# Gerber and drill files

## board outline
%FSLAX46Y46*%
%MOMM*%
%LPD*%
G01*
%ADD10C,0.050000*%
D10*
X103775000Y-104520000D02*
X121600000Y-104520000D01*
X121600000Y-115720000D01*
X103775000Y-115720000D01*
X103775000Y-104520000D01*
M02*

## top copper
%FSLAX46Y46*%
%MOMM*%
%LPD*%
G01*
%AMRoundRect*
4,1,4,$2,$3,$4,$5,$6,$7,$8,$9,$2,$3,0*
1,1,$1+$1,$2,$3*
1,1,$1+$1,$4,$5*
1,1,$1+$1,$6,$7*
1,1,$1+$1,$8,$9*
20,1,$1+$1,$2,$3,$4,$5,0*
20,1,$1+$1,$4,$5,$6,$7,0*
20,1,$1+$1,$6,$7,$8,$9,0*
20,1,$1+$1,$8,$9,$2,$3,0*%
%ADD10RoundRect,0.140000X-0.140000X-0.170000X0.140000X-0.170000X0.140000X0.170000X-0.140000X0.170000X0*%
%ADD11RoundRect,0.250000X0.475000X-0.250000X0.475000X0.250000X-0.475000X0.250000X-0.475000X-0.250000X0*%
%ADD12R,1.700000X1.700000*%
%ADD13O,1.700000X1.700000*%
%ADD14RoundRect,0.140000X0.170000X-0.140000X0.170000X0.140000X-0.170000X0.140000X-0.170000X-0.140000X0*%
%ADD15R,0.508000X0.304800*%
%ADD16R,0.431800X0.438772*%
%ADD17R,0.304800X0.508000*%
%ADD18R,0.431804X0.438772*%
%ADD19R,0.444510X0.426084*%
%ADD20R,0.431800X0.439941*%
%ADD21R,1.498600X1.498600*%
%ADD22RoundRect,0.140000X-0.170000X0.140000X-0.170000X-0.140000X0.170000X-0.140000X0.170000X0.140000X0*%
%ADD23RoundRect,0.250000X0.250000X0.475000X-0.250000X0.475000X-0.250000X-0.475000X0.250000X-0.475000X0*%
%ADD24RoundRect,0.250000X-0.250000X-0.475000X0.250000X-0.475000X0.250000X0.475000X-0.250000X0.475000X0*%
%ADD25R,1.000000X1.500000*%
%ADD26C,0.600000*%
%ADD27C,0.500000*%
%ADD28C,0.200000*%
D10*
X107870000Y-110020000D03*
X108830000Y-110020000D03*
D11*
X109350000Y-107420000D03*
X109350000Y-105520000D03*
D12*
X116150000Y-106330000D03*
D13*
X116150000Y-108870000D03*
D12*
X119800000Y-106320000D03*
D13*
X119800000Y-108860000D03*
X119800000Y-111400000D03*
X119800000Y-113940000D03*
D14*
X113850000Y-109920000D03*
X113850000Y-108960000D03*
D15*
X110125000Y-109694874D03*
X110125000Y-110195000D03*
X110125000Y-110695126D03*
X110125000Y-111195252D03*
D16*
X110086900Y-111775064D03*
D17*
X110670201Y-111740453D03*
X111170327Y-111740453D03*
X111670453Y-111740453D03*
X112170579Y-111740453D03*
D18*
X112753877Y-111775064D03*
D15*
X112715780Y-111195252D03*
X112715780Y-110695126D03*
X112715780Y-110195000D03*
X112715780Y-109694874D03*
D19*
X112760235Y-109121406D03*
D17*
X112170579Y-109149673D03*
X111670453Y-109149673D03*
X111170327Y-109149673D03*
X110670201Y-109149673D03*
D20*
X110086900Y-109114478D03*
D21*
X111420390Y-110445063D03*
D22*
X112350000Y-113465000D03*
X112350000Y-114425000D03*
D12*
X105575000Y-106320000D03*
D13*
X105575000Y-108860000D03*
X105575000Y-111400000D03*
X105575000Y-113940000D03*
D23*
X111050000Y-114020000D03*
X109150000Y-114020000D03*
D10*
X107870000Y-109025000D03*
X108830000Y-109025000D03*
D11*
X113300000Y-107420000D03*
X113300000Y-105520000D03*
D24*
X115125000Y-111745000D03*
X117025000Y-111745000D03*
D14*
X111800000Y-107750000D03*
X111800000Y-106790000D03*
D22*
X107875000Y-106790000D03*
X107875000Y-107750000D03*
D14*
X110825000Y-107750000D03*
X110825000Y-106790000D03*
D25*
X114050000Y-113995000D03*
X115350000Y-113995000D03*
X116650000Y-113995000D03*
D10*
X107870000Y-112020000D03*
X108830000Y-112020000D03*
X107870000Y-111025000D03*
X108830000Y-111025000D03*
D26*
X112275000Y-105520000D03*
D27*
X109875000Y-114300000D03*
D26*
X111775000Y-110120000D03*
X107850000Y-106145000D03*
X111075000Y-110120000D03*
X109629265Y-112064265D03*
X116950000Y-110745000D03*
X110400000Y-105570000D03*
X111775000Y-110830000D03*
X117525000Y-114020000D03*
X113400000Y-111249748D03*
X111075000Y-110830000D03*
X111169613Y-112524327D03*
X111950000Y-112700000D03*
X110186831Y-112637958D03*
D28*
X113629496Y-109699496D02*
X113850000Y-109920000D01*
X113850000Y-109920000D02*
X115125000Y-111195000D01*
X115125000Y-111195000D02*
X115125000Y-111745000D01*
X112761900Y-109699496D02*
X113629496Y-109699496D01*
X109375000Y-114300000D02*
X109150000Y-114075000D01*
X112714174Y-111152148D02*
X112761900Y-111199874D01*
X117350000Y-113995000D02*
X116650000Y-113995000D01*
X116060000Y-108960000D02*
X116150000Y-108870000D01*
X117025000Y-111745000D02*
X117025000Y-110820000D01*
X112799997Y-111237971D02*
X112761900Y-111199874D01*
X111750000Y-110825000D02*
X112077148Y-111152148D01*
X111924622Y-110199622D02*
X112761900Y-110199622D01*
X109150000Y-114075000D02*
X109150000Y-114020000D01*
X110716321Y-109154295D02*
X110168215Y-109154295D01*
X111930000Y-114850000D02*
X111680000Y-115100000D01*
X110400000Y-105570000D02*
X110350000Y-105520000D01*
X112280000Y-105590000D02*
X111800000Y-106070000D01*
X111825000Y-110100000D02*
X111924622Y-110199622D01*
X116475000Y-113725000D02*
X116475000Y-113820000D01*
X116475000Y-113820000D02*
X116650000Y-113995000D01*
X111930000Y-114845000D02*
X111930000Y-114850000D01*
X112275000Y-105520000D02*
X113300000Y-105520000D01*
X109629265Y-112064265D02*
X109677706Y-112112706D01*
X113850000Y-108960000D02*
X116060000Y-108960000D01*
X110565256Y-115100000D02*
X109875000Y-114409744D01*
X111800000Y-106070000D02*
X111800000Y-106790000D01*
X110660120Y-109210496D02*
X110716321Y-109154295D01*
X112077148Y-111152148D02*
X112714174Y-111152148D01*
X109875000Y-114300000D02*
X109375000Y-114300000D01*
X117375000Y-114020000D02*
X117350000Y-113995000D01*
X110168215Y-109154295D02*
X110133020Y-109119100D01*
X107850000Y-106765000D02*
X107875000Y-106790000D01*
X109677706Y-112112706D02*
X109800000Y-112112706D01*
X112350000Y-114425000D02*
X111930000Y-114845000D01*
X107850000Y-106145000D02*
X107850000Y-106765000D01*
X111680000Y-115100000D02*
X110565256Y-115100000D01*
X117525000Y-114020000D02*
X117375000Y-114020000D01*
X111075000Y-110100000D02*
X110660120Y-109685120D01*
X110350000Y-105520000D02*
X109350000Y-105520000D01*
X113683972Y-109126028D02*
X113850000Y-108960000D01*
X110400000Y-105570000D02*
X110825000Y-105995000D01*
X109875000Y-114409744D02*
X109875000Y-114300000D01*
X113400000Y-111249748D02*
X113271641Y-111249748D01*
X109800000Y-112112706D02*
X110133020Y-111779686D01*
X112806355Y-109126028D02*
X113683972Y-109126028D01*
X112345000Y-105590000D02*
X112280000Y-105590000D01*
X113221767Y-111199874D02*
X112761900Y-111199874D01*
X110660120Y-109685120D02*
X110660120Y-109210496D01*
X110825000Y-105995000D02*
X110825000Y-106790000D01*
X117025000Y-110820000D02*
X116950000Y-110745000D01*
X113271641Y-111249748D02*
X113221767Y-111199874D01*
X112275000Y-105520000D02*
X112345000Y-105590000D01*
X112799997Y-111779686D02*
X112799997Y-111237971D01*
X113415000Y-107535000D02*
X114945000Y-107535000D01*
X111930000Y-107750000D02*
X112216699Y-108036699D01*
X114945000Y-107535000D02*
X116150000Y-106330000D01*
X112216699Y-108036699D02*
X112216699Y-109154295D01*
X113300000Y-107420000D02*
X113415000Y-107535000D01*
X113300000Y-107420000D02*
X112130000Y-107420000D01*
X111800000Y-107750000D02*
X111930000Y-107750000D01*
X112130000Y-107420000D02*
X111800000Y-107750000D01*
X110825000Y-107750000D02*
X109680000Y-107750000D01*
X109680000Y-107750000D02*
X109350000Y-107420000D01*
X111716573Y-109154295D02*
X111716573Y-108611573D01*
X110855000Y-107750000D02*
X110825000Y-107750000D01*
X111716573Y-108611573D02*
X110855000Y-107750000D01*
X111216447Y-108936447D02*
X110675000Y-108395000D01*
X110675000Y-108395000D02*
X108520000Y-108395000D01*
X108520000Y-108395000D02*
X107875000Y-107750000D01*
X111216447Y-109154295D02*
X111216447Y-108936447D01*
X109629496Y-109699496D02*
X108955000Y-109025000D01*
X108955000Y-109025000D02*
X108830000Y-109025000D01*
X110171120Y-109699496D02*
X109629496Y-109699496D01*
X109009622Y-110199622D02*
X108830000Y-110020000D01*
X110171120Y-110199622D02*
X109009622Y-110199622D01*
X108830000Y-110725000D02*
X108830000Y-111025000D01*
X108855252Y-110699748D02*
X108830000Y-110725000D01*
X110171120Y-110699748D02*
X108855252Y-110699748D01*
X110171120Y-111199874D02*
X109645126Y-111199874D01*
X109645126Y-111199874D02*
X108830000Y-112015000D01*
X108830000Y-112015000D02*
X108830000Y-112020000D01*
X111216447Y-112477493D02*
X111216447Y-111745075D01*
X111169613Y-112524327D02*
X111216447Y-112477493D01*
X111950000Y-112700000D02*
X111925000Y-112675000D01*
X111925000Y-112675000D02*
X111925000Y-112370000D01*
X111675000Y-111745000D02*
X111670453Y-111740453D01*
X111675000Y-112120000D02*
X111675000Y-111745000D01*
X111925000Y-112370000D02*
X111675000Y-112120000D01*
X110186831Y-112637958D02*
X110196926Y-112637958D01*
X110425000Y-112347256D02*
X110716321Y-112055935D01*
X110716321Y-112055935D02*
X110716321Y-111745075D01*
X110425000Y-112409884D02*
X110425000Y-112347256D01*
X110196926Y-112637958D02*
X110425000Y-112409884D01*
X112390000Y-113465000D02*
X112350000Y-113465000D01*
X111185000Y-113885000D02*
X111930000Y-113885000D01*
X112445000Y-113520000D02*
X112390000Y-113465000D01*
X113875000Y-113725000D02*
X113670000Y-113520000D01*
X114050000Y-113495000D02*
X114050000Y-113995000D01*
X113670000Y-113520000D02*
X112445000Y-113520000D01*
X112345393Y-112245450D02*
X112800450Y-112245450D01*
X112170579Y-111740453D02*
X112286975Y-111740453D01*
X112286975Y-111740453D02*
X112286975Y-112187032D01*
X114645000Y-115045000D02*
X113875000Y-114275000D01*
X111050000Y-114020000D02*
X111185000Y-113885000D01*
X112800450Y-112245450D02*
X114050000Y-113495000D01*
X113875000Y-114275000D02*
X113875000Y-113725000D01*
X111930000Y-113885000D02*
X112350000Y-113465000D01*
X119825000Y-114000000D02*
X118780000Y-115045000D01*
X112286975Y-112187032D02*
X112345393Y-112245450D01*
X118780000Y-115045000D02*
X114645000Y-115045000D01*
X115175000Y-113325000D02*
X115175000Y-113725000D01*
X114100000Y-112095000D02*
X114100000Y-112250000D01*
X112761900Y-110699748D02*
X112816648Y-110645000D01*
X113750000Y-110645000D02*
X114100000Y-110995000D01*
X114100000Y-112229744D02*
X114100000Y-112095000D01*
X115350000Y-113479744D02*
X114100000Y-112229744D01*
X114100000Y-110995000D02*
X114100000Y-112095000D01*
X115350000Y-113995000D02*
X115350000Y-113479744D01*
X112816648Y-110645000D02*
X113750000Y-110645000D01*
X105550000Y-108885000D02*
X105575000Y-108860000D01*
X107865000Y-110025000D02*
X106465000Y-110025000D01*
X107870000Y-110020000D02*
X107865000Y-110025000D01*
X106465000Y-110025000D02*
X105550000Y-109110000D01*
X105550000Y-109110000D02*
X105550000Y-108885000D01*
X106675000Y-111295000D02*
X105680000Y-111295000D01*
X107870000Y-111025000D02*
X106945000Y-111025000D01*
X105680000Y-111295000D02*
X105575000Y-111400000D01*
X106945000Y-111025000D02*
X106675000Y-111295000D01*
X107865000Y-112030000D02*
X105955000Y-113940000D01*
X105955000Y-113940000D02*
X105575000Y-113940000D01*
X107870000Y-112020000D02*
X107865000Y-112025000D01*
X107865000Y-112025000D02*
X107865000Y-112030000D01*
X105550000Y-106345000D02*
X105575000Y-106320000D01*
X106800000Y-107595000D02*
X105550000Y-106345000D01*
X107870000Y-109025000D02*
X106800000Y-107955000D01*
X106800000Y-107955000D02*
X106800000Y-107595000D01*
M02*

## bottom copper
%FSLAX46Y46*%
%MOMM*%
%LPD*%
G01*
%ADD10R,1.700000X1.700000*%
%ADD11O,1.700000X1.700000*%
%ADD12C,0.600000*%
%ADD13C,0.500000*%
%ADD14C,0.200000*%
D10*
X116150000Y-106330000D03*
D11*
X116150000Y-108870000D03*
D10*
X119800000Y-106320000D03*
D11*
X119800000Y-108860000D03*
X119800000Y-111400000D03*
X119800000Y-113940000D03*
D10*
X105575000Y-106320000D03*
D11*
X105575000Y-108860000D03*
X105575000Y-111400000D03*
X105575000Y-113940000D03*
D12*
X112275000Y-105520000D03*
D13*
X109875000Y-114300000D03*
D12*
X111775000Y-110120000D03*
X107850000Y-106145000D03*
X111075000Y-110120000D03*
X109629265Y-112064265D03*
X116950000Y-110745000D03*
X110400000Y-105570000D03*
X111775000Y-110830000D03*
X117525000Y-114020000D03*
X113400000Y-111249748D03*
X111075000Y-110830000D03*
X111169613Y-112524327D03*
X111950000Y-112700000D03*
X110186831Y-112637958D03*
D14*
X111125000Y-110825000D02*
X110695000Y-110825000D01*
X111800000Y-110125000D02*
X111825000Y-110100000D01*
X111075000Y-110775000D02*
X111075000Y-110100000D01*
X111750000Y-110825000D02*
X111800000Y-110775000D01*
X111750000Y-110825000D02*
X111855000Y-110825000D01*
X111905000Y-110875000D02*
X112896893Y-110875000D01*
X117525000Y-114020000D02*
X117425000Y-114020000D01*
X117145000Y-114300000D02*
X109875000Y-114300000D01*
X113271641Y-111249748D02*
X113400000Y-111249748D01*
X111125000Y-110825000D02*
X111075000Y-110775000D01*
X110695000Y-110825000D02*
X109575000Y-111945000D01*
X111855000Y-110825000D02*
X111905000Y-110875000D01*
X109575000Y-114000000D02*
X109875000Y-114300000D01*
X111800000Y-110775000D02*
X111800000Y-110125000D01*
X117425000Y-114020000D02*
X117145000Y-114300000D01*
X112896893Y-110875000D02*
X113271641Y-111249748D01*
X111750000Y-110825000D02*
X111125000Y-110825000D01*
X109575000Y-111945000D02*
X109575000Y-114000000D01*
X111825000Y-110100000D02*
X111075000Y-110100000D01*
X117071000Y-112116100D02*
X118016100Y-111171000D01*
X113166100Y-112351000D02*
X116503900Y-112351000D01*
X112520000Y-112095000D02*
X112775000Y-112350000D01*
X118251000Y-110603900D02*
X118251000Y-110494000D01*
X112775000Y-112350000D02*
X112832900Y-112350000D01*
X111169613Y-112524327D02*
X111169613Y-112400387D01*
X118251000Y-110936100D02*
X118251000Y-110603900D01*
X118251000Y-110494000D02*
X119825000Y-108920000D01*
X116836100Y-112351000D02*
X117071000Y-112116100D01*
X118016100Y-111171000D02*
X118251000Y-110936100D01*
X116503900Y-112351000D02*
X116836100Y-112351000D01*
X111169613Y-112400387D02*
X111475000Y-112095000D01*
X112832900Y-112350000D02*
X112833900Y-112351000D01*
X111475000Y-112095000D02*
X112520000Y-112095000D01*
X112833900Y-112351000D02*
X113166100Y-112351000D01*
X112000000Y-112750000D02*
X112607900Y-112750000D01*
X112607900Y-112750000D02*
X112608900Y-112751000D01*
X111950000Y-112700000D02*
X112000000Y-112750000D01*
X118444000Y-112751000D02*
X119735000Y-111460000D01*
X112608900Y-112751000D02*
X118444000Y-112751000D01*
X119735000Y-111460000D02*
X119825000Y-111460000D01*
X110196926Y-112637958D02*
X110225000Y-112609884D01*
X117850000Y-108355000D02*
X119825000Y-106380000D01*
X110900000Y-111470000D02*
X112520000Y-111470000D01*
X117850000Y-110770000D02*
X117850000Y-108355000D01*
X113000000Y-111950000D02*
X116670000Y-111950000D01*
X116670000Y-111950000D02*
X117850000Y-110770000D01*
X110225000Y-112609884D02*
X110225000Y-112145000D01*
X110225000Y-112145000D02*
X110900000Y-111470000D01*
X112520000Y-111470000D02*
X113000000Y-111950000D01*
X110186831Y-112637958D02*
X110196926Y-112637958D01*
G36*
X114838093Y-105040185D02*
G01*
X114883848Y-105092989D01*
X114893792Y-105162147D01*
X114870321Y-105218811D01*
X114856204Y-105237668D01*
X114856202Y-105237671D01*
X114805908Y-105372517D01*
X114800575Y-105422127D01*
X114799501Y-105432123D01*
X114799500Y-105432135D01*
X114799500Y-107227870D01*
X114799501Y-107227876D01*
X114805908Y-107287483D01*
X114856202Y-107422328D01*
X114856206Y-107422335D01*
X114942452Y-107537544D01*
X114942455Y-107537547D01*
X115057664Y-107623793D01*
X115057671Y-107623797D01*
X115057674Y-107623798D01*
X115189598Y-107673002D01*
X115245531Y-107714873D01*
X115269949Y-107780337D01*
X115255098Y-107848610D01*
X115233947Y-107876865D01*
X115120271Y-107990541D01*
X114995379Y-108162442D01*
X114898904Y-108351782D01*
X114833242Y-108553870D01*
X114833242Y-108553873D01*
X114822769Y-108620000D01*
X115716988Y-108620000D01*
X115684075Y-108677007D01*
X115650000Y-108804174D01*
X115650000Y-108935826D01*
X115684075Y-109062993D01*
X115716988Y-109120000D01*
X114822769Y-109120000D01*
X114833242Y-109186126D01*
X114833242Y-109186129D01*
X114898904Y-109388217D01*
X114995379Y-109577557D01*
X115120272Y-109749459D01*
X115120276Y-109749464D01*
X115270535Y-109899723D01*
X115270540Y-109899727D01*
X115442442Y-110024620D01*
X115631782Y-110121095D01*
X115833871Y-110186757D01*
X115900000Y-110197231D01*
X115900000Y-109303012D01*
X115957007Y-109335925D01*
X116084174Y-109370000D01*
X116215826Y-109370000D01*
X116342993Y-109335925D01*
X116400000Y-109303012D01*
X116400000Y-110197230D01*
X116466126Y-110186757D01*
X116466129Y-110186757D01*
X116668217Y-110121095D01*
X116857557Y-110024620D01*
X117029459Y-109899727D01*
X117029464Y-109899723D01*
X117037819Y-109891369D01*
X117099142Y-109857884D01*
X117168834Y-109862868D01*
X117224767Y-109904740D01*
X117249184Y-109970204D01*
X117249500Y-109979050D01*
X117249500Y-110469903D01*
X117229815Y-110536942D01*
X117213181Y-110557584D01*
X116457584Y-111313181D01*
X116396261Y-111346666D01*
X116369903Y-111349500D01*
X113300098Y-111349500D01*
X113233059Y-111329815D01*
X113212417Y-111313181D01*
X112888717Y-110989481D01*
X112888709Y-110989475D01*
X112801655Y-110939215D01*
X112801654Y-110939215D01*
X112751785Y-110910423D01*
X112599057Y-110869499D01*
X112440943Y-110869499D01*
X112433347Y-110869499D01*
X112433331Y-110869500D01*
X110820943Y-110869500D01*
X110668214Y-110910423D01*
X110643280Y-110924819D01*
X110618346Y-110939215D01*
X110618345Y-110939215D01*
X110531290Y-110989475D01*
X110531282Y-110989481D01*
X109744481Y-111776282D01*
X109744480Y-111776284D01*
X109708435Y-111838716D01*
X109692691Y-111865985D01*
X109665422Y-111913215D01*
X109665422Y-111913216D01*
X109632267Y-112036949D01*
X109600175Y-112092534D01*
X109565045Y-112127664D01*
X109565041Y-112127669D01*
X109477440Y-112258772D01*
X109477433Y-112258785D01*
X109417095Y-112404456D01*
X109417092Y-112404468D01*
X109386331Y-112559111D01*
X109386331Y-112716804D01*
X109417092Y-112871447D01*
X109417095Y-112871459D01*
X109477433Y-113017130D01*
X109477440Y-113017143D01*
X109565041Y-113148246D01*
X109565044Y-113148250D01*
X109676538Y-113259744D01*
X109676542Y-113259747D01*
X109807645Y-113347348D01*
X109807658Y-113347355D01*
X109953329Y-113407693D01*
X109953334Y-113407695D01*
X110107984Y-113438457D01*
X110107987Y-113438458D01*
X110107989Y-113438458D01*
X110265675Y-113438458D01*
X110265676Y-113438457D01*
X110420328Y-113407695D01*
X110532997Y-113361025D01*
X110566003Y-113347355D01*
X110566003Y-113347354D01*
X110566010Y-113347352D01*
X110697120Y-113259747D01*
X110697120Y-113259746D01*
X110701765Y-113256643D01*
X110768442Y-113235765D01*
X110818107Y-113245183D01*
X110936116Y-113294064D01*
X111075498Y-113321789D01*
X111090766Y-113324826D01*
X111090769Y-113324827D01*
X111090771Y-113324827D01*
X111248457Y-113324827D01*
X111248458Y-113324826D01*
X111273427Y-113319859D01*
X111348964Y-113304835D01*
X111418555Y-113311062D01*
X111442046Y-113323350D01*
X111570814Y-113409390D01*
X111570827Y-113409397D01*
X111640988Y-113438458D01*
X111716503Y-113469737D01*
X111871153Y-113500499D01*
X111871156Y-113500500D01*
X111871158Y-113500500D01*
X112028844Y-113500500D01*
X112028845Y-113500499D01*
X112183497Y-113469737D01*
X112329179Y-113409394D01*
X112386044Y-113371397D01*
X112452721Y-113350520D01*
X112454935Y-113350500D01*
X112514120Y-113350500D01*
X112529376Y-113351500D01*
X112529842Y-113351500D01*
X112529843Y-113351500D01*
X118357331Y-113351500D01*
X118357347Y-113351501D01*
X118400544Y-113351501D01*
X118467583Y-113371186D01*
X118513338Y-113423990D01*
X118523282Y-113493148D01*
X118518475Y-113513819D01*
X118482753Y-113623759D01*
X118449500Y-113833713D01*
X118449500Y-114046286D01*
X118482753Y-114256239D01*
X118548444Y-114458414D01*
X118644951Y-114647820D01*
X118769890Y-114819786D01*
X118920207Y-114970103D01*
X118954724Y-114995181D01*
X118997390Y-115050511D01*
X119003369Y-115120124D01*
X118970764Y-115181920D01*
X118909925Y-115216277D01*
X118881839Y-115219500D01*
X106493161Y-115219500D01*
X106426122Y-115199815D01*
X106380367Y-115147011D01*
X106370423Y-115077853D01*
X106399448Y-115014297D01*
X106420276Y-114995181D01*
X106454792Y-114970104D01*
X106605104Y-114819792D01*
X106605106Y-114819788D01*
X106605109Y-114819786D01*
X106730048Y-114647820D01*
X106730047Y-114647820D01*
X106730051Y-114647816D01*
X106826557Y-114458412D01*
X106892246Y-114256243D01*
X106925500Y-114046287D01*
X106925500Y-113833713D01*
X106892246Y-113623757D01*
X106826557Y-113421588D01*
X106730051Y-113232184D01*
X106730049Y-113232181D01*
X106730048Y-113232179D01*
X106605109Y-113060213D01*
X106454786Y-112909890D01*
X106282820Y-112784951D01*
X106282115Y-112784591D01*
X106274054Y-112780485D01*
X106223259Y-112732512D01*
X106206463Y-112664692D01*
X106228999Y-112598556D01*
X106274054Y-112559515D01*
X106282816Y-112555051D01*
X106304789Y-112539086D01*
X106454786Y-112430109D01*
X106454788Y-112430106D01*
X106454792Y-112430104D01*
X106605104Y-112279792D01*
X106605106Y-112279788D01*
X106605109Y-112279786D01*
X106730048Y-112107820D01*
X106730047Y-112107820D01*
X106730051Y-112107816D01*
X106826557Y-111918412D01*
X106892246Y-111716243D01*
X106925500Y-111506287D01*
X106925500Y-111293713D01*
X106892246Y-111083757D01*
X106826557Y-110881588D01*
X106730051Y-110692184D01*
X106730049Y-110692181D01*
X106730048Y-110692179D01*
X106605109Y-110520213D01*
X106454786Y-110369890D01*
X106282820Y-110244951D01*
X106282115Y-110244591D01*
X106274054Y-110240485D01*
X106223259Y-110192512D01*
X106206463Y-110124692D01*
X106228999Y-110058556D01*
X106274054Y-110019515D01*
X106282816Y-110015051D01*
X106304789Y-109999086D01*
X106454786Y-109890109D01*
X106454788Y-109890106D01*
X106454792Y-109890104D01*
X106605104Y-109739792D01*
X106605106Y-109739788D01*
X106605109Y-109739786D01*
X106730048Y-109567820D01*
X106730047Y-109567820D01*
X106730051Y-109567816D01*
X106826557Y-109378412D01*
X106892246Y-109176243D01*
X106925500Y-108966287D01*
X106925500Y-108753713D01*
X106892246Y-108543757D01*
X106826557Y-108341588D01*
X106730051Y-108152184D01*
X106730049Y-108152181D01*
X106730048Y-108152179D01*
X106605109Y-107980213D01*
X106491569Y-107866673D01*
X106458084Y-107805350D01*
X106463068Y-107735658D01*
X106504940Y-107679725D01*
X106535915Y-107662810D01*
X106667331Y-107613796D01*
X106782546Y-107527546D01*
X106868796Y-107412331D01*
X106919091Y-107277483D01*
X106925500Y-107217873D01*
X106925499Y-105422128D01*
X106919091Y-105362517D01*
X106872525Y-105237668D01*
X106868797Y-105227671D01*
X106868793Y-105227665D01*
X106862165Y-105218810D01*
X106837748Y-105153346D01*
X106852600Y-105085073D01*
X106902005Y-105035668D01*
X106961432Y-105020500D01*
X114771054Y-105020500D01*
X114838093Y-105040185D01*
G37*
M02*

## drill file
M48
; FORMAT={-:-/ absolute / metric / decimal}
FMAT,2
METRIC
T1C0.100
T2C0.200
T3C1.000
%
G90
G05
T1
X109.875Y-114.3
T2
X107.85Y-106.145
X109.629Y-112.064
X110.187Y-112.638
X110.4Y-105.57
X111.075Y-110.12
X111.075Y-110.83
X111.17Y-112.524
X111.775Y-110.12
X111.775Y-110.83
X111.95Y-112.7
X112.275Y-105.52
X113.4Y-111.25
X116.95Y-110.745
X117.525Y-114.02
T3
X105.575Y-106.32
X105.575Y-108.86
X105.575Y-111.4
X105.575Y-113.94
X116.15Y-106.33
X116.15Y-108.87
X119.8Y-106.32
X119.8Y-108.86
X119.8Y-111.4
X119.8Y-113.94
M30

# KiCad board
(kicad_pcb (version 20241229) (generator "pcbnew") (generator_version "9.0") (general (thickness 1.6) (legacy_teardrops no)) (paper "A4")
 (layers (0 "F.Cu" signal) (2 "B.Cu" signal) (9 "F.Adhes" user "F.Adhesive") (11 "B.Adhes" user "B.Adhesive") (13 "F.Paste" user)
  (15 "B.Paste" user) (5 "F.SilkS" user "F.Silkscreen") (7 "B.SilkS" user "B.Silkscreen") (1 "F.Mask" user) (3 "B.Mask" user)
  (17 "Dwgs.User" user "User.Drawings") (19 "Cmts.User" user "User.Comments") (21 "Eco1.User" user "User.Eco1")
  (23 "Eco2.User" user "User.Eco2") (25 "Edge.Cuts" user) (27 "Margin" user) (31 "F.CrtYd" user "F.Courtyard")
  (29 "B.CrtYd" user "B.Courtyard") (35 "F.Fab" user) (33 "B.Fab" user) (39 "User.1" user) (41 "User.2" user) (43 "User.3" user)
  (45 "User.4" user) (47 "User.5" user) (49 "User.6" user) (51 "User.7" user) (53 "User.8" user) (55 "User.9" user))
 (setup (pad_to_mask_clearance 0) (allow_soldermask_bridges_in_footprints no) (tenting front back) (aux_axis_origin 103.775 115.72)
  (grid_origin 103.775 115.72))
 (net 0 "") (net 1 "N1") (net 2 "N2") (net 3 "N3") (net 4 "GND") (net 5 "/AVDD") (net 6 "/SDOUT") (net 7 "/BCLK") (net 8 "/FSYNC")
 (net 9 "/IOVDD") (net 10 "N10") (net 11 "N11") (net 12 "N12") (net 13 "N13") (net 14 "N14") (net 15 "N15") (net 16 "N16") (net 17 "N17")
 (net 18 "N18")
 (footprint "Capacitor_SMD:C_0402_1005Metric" (layer "F.Cu") (at 108.35 110.02)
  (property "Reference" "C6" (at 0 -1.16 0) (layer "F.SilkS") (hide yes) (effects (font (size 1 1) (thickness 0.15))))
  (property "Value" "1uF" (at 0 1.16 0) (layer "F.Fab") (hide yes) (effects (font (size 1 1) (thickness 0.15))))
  (pad "1" smd roundrect (at -0.48 0) (size 0.56 0.62) (layers "F.Cu" "F.Mask" "F.Paste") (roundrect_rratio 0.25) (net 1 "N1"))
  (pad "2" smd roundrect (at 0.48 0) (size 0.56 0.62) (layers "F.Cu" "F.Mask" "F.Paste") (roundrect_rratio 0.25) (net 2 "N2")))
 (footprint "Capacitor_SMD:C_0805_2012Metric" (layer "F.Cu") (at 109.35 106.47 90)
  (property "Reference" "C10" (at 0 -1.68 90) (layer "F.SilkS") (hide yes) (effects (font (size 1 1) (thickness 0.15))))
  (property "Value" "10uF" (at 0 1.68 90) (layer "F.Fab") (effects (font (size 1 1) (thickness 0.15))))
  (pad "1" smd roundrect (at -0.95 0 90) (size 1 1.45) (layers "F.Cu" "F.Mask" "F.Paste") (roundrect_rratio 0.25) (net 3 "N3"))
  (pad "2" smd roundrect (at 0.95 0 90) (size 1 1.45) (layers "F.Cu" "F.Mask" "F.Paste") (roundrect_rratio 0.25) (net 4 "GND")))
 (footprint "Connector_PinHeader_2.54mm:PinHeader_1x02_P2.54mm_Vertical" (layer "F.Cu") (at 116.15 106.33)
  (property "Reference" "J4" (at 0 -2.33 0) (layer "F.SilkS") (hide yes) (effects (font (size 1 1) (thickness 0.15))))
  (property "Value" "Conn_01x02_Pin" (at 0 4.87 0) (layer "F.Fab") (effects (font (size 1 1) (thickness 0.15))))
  (pad "1" thru_hole rect (at 0 0) (size 1.7 1.7) (drill 1) (layers "*.Cu" "*.Mask") (remove_unused_layers no) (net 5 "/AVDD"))
  (pad "2" thru_hole oval (at 0 2.54) (size 1.7 1.7) (drill 1) (layers "*.Cu" "*.Mask") (remove_unused_layers no) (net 4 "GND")))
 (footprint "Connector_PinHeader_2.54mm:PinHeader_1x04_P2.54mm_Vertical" (layer "F.Cu") (at 119.8 106.32)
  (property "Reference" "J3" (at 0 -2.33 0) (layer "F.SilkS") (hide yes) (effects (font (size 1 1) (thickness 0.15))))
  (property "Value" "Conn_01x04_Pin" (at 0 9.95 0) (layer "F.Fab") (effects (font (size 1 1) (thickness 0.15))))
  (pad "1" thru_hole rect (at 0 0) (size 1.7 1.7) (drill 1) (layers "*.Cu" "*.Mask") (remove_unused_layers no) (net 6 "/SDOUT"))
  (pad "2" thru_hole oval (at 0 2.54) (size 1.7 1.7) (drill 1) (layers "*.Cu" "*.Mask") (remove_unused_layers no) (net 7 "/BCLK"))
  (pad "3" thru_hole oval (at 0 5.08) (size 1.7 1.7) (drill 1) (layers "*.Cu" "*.Mask") (remove_unused_layers no) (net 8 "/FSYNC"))
  (pad "4" thru_hole oval (at 0 7.62) (size 1.7 1.7) (drill 1) (layers "*.Cu" "*.Mask") (remove_unused_layers no) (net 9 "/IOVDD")))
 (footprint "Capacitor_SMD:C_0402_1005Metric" (layer "F.Cu") (at 113.85 109.44 90)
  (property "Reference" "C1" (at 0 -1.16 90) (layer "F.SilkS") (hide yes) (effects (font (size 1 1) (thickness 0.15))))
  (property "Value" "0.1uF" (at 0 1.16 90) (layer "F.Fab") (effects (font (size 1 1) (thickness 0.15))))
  (pad "1" smd roundrect (at -0.48 0 90) (size 0.56 0.62) (layers "F.Cu" "F.Mask" "F.Paste") (roundrect_rratio 0.25) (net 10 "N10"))
  (pad "2" smd roundrect (at 0.48 0 90) (size 0.56 0.62) (layers "F.Cu" "F.Mask" "F.Paste") (roundrect_rratio 0.25) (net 4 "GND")))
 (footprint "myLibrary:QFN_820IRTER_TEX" (layer "F.Cu") (at 111.42039 110.445063)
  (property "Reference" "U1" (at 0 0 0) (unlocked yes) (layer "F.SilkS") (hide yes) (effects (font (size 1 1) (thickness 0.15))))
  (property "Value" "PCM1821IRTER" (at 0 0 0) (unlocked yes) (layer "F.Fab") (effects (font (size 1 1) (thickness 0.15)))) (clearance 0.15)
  (pad "1" smd rect (at -1.29539 -0.750189 90) (size 0.3048 0.508) (layers "F.Cu" "F.Mask" "F.Paste") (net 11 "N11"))
  (pad "2" smd rect (at -1.29539 -0.250063 90) (size 0.3048 0.508) (layers "F.Cu" "F.Mask" "F.Paste") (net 2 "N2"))
  (pad "3" smd rect (at -1.29539 0.250063 90) (size 0.3048 0.508) (layers "F.Cu" "F.Mask" "F.Paste") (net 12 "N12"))
  (pad "4" smd rect (at -1.29539 0.750189 90) (size 0.3048 0.508) (layers "F.Cu" "F.Mask" "F.Paste") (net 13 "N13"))
  (pad "5" smd rect (at -1.33349 1.330001 90) (size 0.438772 0.4318) (layers "F.Cu" "F.Mask" "F.Paste") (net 4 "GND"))
  (pad "6" smd rect (at -0.750189 1.29539) (size 0.3048 0.508) (layers "F.Cu" "F.Mask" "F.Paste") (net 6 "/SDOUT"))
  (pad "7" smd rect (at -0.250063 1.29539) (size 0.3048 0.508) (layers "F.Cu" "F.Mask" "F.Paste") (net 7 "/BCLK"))
  (pad "8" smd rect (at 0.250063 1.29539) (size 0.3048 0.508) (layers "F.Cu" "F.Mask" "F.Paste") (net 8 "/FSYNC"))
  (pad "9" smd rect (at 0.750189 1.29539) (size 0.3048 0.508) (layers "F.Cu" "F.Mask" "F.Paste") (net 9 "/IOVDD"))
  (pad "10" smd rect (at 1.333487 1.330001 90) (size 0.438772 0.431804) (layers "F.Cu" "F.Mask" "F.Paste") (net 4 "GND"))
  (pad "11" smd rect (at 1.29539 0.750189 90) (size 0.3048 0.508) (layers "F.Cu" "F.Mask" "F.Paste") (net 4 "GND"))
  (pad "12" smd rect (at 1.29539 0.250063 90) (size 0.3048 0.508) (layers "F.Cu" "F.Mask" "F.Paste") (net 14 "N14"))
  (pad "13" smd rect (at 1.29539 -0.250063 90) (size 0.3048 0.508) (layers "F.Cu" "F.Mask" "F.Paste") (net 4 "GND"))
  (pad "14" smd rect (at 1.29539 -0.750189 90) (size 0.3048 0.508) (layers "F.Cu" "F.Mask" "F.Paste") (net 10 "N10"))
  (pad "15" smd rect (at 1.339845 -1.323657 90) (size 0.426084 0.44451) (layers "F.Cu" "F.Mask" "F.Paste") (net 4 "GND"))
  (pad "16" smd rect (at 0.750189 -1.29539) (size 0.3048 0.508) (layers "F.Cu" "F.Mask" "F.Paste") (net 5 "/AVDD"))
  (pad "17" smd rect (at 0.250063 -1.29539) (size 0.3048 0.508) (layers "F.Cu" "F.Mask" "F.Paste") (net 3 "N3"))
  (pad "18" smd rect (at -0.250063 -1.29539) (size 0.3048 0.508) (layers "F.Cu" "F.Mask" "F.Paste") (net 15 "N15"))
  (pad "19" smd rect (at -0.750189 -1.29539) (size 0.3048 0.508) (layers "F.Cu" "F.Mask" "F.Paste") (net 4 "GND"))
  (pad "20" smd rect (at -1.33349 -1.330585 90) (size 0.439941 0.4318) (layers "F.Cu" "F.Mask" "F.Paste") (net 4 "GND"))
  (pad "21" smd rect (at 0 0) (size 1.4986 1.4986) (layers "F.Cu" "F.Mask" "F.Paste") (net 4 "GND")))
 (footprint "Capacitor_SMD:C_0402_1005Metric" (layer "F.Cu") (at 112.35 113.945 -90)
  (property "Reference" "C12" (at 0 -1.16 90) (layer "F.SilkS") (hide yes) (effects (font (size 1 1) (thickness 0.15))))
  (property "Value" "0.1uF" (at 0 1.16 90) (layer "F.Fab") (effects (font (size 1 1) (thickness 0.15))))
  (pad "1" smd roundrect (at -0.48 0 270) (size 0.56 0.62) (layers "F.Cu" "F.Mask" "F.Paste") (roundrect_rratio 0.25) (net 9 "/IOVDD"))
  (pad "2" smd roundrect (at 0.48 0 270) (size 0.56 0.62) (layers "F.Cu" "F.Mask" "F.Paste") (roundrect_rratio 0.25) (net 4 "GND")))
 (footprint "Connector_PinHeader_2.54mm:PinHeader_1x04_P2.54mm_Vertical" (layer "F.Cu") (at 105.575 106.32)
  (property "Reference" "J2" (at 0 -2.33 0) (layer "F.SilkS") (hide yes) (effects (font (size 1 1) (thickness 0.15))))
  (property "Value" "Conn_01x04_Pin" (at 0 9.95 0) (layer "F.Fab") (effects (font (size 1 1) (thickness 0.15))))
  (pad "1" thru_hole rect (at 0 0) (size 1.7 1.7) (drill 1) (layers "*.Cu" "*.Mask") (remove_unused_layers no) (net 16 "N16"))
  (pad "2" thru_hole oval (at 0 2.54) (size 1.7 1.7) (drill 1) (layers "*.Cu" "*.Mask") (remove_unused_layers no) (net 1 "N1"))
  (pad "3" thru_hole oval (at 0 5.08) (size 1.7 1.7) (drill 1) (layers "*.Cu" "*.Mask") (remove_unused_layers no) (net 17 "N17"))
  (pad "4" thru_hole oval (at 0 7.62) (size 1.7 1.7) (drill 1) (layers "*.Cu" "*.Mask") (remove_unused_layers no) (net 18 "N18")))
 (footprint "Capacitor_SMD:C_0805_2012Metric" (layer "F.Cu") (at 110.1 114.02 180)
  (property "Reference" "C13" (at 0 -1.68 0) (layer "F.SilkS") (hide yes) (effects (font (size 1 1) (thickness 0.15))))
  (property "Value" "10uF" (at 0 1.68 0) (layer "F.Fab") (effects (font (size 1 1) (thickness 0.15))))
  (pad "1" smd roundrect (at -0.95 0 180) (size 1 1.45) (layers "F.Cu" "F.Mask" "F.Paste") (roundrect_rratio 0.25) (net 9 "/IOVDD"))
  (pad "2" smd roundrect (at 0.95 0 180) (size 1 1.45) (layers "F.Cu" "F.Mask" "F.Paste") (roundrect_rratio 0.25) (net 4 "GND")))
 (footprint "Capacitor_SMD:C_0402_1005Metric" (layer "F.Cu") (at 108.35 109.025)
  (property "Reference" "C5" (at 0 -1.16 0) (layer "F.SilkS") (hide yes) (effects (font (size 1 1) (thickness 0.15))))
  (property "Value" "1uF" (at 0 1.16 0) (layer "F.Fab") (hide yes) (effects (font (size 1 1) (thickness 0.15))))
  (pad "1" smd roundrect (at -0.48 0) (size 0.56 0.62) (layers "F.Cu" "F.Mask" "F.Paste") (roundrect_rratio 0.25) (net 16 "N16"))
  (pad "2" smd roundrect (at 0.48 0) (size 0.56 0.62) (layers "F.Cu" "F.Mask" "F.Paste") (roundrect_rratio 0.25) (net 11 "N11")))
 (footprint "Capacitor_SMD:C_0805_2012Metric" (layer "F.Cu") (at 113.3 106.47 90)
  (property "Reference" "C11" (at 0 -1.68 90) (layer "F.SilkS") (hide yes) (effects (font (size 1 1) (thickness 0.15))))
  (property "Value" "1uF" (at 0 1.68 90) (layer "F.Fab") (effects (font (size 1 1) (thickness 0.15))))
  (pad "1" smd roundrect (at -0.95 0 90) (size 1 1.45) (layers "F.Cu" "F.Mask" "F.Paste") (roundrect_rratio 0.25) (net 5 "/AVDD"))
  (pad "2" smd roundrect (at 0.95 0 90) (size 1 1.45) (layers "F.Cu" "F.Mask" "F.Paste") (roundrect_rratio 0.25) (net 4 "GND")))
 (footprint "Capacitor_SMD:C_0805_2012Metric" (layer "F.Cu") (at 116.075 111.745)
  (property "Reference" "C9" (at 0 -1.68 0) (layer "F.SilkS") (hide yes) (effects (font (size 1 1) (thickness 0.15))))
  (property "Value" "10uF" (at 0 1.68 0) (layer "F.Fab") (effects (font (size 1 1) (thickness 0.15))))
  (pad "1" smd roundrect (at -0.95 0) (size 1 1.45) (layers "F.Cu" "F.Mask" "F.Paste") (roundrect_rratio 0.25) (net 10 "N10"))
  (pad "2" smd roundrect (at 0.95 0) (size 1 1.45) (layers "F.Cu" "F.Mask" "F.Paste") (roundrect_rratio 0.25) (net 4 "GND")))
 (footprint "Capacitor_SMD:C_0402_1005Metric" (layer "F.Cu") (at 111.8 107.27 90)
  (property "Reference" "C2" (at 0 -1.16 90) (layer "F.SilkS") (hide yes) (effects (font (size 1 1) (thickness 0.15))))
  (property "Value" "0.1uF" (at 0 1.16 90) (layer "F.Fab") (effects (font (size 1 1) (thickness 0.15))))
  (pad "1" smd roundrect (at -0.48 0 90) (size 0.56 0.62) (layers "F.Cu" "F.Mask" "F.Paste") (roundrect_rratio 0.25) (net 5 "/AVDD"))
  (pad "2" smd roundrect (at 0.48 0 90) (size 0.56 0.62) (layers "F.Cu" "F.Mask" "F.Paste") (roundrect_rratio 0.25) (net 4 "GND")))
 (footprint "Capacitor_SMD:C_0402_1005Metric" (layer "F.Cu") (at 107.875 107.27 -90)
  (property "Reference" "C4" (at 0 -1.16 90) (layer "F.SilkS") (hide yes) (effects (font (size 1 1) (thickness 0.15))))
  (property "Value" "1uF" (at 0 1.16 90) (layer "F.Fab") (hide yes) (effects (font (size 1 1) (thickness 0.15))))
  (pad "1" smd roundrect (at -0.48 0 270) (size 0.56 0.62) (layers "F.Cu" "F.Mask" "F.Paste") (roundrect_rratio 0.25) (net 4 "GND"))
  (pad "2" smd roundrect (at 0.48 0 270) (size 0.56 0.62) (layers "F.Cu" "F.Mask" "F.Paste") (roundrect_rratio 0.25) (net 15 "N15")))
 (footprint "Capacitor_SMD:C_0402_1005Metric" (layer "F.Cu") (at 110.825 107.27 90)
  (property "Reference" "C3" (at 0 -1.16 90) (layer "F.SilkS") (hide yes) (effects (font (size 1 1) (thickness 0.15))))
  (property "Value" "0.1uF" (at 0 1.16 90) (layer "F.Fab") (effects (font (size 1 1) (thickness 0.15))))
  (pad "1" smd roundrect (at -0.48 0 90) (size 0.56 0.62) (layers "F.Cu" "F.Mask" "F.Paste") (roundrect_rratio 0.25) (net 3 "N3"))
  (pad "2" smd roundrect (at 0.48 0 90) (size 0.56 0.62) (layers "F.Cu" "F.Mask" "F.Paste") (roundrect_rratio 0.25) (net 4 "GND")))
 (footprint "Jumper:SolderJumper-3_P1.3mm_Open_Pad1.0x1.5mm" (layer "F.Cu") (at 115.35 113.995)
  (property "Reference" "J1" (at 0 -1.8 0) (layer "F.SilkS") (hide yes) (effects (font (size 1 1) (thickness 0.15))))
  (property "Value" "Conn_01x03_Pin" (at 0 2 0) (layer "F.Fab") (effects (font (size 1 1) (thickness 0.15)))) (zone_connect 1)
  (pad "1" smd rect (at -1.3 0) (size 1 1.5) (layers "F.Cu" "F.Mask") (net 9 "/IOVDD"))
  (pad "2" smd rect (at 0 0) (size 1 1.5) (layers "F.Cu" "F.Mask") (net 14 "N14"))
  (pad "3" smd rect (at 1.3 0) (size 1 1.5) (layers "F.Cu" "F.Mask") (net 4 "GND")))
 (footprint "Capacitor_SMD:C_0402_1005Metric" (layer "F.Cu") (at 108.35 112.02)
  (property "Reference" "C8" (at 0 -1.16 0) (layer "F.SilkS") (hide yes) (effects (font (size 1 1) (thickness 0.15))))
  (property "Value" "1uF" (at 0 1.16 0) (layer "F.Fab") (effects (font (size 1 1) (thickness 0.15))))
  (pad "1" smd roundrect (at -0.48 0) (size 0.56 0.62) (layers "F.Cu" "F.Mask" "F.Paste") (roundrect_rratio 0.25) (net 18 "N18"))
  (pad "2" smd roundrect (at 0.48 0) (size 0.56 0.62) (layers "F.Cu" "F.Mask" "F.Paste") (roundrect_rratio 0.25) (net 13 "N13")))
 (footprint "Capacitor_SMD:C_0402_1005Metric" (layer "F.Cu") (at 108.35 111.025)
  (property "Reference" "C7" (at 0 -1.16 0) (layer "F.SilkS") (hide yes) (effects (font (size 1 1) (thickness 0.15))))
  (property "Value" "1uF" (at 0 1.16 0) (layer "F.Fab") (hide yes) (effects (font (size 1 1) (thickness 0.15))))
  (pad "1" smd roundrect (at -0.48 0) (size 0.56 0.62) (layers "F.Cu" "F.Mask" "F.Paste") (roundrect_rratio 0.25) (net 17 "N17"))
  (pad "2" smd roundrect (at 0.48 0) (size 0.56 0.62) (layers "F.Cu" "F.Mask" "F.Paste") (roundrect_rratio 0.25) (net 12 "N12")))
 (gr_rect (start 103.775 104.52) (end 121.6 115.72) (stroke (width 0.05) (type default)) (fill no) (layer "Edge.Cuts"))
 (segment (start 113.629496 109.699496) (end 113.85 109.92) (width 0.2) (layer "F.Cu") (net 10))
 (segment (start 113.85 109.92) (end 115.125 111.195) (width 0.2) (layer "F.Cu") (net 10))
 (segment (start 115.125 111.195) (end 115.125 111.745) (width 0.2) (layer "F.Cu") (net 10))
 (segment (start 112.7619 109.699496) (end 113.629496 109.699496) (width 0.2) (layer "F.Cu") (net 10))
 (segment (start 109.375 114.3) (end 109.15 114.075) (width 0.2) (layer "F.Cu") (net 4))
 (segment (start 112.714174 111.152148) (end 112.7619 111.199874) (width 0.2) (layer "F.Cu") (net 4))
 (segment (start 117.35 113.995) (end 116.65 113.995) (width 0.2) (layer "F.Cu") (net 4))
 (segment (start 116.06 108.96) (end 116.15 108.87) (width 0.2) (layer "F.Cu") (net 4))
 (segment (start 117.025 111.745) (end 117.025 110.82) (width 0.2) (layer "F.Cu") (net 4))
 (segment (start 112.799997 111.237971) (end 112.7619 111.199874) (width 0.2) (layer "F.Cu") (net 4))
 (segment (start 111.75 110.825) (end 112.077148 111.152148) (width 0.2) (layer "F.Cu") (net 4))
 (segment (start 111.924622 110.199622) (end 112.7619 110.199622) (width 0.2) (layer "F.Cu") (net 4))
 (segment (start 109.15 114.075) (end 109.15 114.02) (width 0.2) (layer "F.Cu") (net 4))
 (segment (start 110.716321 109.154295) (end 110.168215 109.154295) (width 0.2) (layer "F.Cu") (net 4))
 (segment (start 111.93 114.85) (end 111.68 115.1) (width 0.2) (layer "F.Cu") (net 4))
 (segment (start 110.4 105.57) (end 110.35 105.52) (width 0.2) (layer "F.Cu") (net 4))
 (segment (start 112.28 105.59) (end 111.8 106.07) (width 0.2) (layer "F.Cu") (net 4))
 (segment (start 111.825 110.1) (end 111.924622 110.199622) (width 0.2) (layer "F.Cu") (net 4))
 (segment (start 116.475 113.725) (end 116.475 113.82) (width 0.2) (layer "F.Cu") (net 4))
 (segment (start 116.475 113.82) (end 116.65 113.995) (width 0.2) (layer "F.Cu") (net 4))
 (segment (start 111.93 114.845) (end 111.93 114.85) (width 0.2) (layer "F.Cu") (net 4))
 (segment (start 112.275 105.52) (end 113.3 105.52) (width 0.2) (layer "F.Cu") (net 4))
 (segment (start 109.629265 112.064265) (end 109.677706 112.112706) (width 0.2) (layer "F.Cu") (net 4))
 (segment (start 113.85 108.96) (end 116.06 108.96) (width 0.2) (layer "F.Cu") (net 4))
 (segment (start 110.565256 115.1) (end 109.875 114.409744) (width 0.2) (layer "F.Cu") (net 4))
 (segment (start 111.8 106.07) (end 111.8 106.79) (width 0.2) (layer "F.Cu") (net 4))
 (segment (start 110.66012 109.210496) (end 110.716321 109.154295) (width 0.2) (layer "F.Cu") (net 4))
 (segment (start 112.077148 111.152148) (end 112.714174 111.152148) (width 0.2) (layer "F.Cu") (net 4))
 (segment (start 109.875 114.3) (end 109.375 114.3) (width 0.2) (layer "F.Cu") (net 4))
 (segment (start 117.375 114.02) (end 117.35 113.995) (width 0.2) (layer "F.Cu") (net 4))
 (segment (start 110.168215 109.154295) (end 110.13302 109.1191) (width 0.2) (layer "F.Cu") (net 4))
 (segment (start 107.85 106.765) (end 107.875 106.79) (width 0.2) (layer "F.Cu") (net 4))
 (segment (start 109.677706 112.112706) (end 109.8 112.112706) (width 0.2) (layer "F.Cu") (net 4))
 (segment (start 112.35 114.425) (end 111.93 114.845) (width 0.2) (layer "F.Cu") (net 4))
 (segment (start 107.85 106.145) (end 107.85 106.765) (width 0.2) (layer "F.Cu") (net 4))
 (segment (start 111.68 115.1) (end 110.565256 115.1) (width 0.2) (layer "F.Cu") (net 4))
 (segment (start 117.525 114.02) (end 117.375 114.02) (width 0.2) (layer "F.Cu") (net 4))
 (segment (start 111.075 110.1) (end 110.66012 109.68512) (width 0.2) (layer "F.Cu") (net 4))
 (segment (start 110.35 105.52) (end 109.35 105.52) (width 0.2) (layer "F.Cu") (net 4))
 (segment (start 113.683972 109.126028) (end 113.85 108.96) (width 0.2) (layer "F.Cu") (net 4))
 (segment (start 110.4 105.57) (end 110.825 105.995) (width 0.2) (layer "F.Cu") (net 4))
 (segment (start 109.875 114.409744) (end 109.875 114.3) (width 0.2) (layer "F.Cu") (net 4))
 (segment (start 113.4 111.249748) (end 113.271641 111.249748) (width 0.2) (layer "F.Cu") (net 4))
 (segment (start 109.8 112.112706) (end 110.13302 111.779686) (width 0.2) (layer "F.Cu") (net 4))
 (segment (start 112.806355 109.126028) (end 113.683972 109.126028) (width 0.2) (layer "F.Cu") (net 4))
 (segment (start 112.345 105.59) (end 112.28 105.59) (width 0.2) (layer "F.Cu") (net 4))
 (segment (start 113.221767 111.199874) (end 112.7619 111.199874) (width 0.2) (layer "F.Cu") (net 4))
 (segment (start 110.66012 109.68512) (end 110.66012 109.210496) (width 0.2) (layer "F.Cu") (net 4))
 (segment (start 110.825 105.995) (end 110.825 106.79) (width 0.2) (layer "F.Cu") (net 4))
 (segment (start 117.025 110.82) (end 116.95 110.745) (width 0.2) (layer "F.Cu") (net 4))
 (segment (start 113.271641 111.249748) (end 113.221767 111.199874) (width 0.2) (layer "F.Cu") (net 4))
 (segment (start 112.275 105.52) (end 112.345 105.59) (width 0.2) (layer "F.Cu") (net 4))
 (segment (start 112.799997 111.779686) (end 112.799997 111.237971) (width 0.2) (layer "F.Cu") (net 4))
 (via (at 112.275 105.52) (size 0.6) (drill 0.2) (layers "F.Cu" "B.Cu") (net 4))
 (via (at 109.875 114.3) (size 0.5) (drill 0.1) (layers "F.Cu" "B.Cu") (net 4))
 (via (at 111.775 110.12) (size 0.6) (drill 0.2) (layers "F.Cu" "B.Cu") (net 4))
 (via (at 107.85 106.145) (size 0.6) (drill 0.2) (layers "F.Cu" "B.Cu") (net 4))
 (via (at 111.075 110.12) (size 0.6) (drill 0.2) (layers "F.Cu" "B.Cu") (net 4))
 (via (at 109.629265 112.064265) (size 0.6) (drill 0.2) (layers "F.Cu" "B.Cu") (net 4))
 (via (at 116.95 110.745) (size 0.6) (drill 0.2) (layers "F.Cu" "B.Cu") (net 4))
 (via (at 110.4 105.57) (size 0.6) (drill 0.2) (layers "F.Cu" "B.Cu") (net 4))
 (via (at 111.775 110.83) (size 0.6) (drill 0.2) (layers "F.Cu" "B.Cu") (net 4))
 (via (at 117.525 114.02) (size 0.6) (drill 0.2) (layers "F.Cu" "B.Cu") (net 4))
 (via (at 113.4 111.249748) (size 0.6) (drill 0.2) (layers "F.Cu" "B.Cu") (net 4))
 (via (at 111.075 110.83) (size 0.6) (drill 0.2) (layers "F.Cu" "B.Cu") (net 4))
 (segment (start 111.125 110.825) (end 110.695 110.825) (width 0.2) (layer "B.Cu") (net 4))
 (segment (start 111.8 110.125) (end 111.825 110.1) (width 0.2) (layer "B.Cu") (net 4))
 (segment (start 111.075 110.775) (end 111.075 110.1) (width 0.2) (layer "B.Cu") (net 4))
 (segment (start 111.75 110.825) (end 111.8 110.775) (width 0.2) (layer "B.Cu") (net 4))
 (segment (start 111.75 110.825) (end 111.855 110.825) (width 0.2) (layer "B.Cu") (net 4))
 (segment (start 111.905 110.875) (end 112.896893 110.875) (width 0.2) (layer "B.Cu") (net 4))
 (segment (start 117.525 114.02) (end 117.425 114.02) (width 0.2) (layer "B.Cu") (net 4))
 (segment (start 117.145 114.3) (end 109.875 114.3) (width 0.2) (layer "B.Cu") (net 4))
 (segment (start 113.271641 111.249748) (end 113.4 111.249748) (width 0.2) (layer "B.Cu") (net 4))
 (segment (start 111.125 110.825) (end 111.075 110.775) (width 0.2) (layer "B.Cu") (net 4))
 (segment (start 110.695 110.825) (end 109.575 111.945) (width 0.2) (layer "B.Cu") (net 4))
 (segment (start 111.855 110.825) (end 111.905 110.875) (width 0.2) (layer "B.Cu") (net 4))
 (segment (start 109.575 114) (end 109.875 114.3) (width 0.2) (layer "B.Cu") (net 4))
 (segment (start 111.8 110.775) (end 111.8 110.125) (width 0.2) (layer "B.Cu") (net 4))
 (segment (start 117.425 114.02) (end 117.145 114.3) (width 0.2) (layer "B.Cu") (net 4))
 (segment (start 112.896893 110.875) (end 113.271641 111.249748) (width 0.2) (layer "B.Cu") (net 4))
 (segment (start 111.75 110.825) (end 111.125 110.825) (width 0.2) (layer "B.Cu") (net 4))
 (segment (start 109.575 111.945) (end 109.575 114) (width 0.2) (layer "B.Cu") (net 4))
 (segment (start 111.825 110.1) (end 111.075 110.1) (width 0.2) (layer "B.Cu") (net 4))
 (segment (start 113.415 107.535) (end 114.945 107.535) (width 0.2) (layer "F.Cu") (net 5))
 (segment (start 111.93 107.75) (end 112.216699 108.036699) (width 0.2) (layer "F.Cu") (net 5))
 (segment (start 114.945 107.535) (end 116.15 106.33) (width 0.2) (layer "F.Cu") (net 5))
 (segment (start 112.216699 108.036699) (end 112.216699 109.154295) (width 0.2) (layer "F.Cu") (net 5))
 (segment (start 113.3 107.42) (end 113.415 107.535) (width 0.2) (layer "F.Cu") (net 5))
 (segment (start 113.3 107.42) (end 112.13 107.42) (width 0.2) (layer "F.Cu") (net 5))
 (segment (start 111.8 107.75) (end 111.93 107.75) (width 0.2) (layer "F.Cu") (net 5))
 (segment (start 112.13 107.42) (end 111.8 107.75) (width 0.2) (layer "F.Cu") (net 5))
 (segment (start 110.825 107.75) (end 109.68 107.75) (width 0.2) (layer "F.Cu") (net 3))
 (segment (start 109.68 107.75) (end 109.35 107.42) (width 0.2) (layer "F.Cu") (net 3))
 (segment (start 111.716573 109.154295) (end 111.716573 108.611573) (width 0.2) (layer "F.Cu") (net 3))
 (segment (start 110.855 107.75) (end 110.825 107.75) (width 0.2) (layer "F.Cu") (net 3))
 (segment (start 111.716573 108.611573) (end 110.855 107.75) (width 0.2) (layer "F.Cu") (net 3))
 (segment (start 111.216447 108.936447) (end 110.675 108.395) (width 0.2) (layer "F.Cu") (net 15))
 (segment (start 110.675 108.395) (end 108.52 108.395) (width 0.2) (layer "F.Cu") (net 15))
 (segment (start 108.52 108.395) (end 107.875 107.75) (width 0.2) (layer "F.Cu") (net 15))
 (segment (start 111.216447 109.154295) (end 111.216447 108.936447) (width 0.2) (layer "F.Cu") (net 15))
 (segment (start 109.629496 109.699496) (end 108.955 109.025) (width 0.2) (layer "F.Cu") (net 11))
 (segment (start 108.955 109.025) (end 108.83 109.025) (width 0.2) (layer "F.Cu") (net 11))
 (segment (start 110.17112 109.699496) (end 109.629496 109.699496) (width 0.2) (layer "F.Cu") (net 11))
 (segment (start 109.009622 110.199622) (end 108.83 110.02) (width 0.2) (layer "F.Cu") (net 2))
 (segment (start 110.17112 110.199622) (end 109.009622 110.199622) (width 0.2) (layer "F.Cu") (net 2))
 (segment (start 108.83 110.725) (end 108.83 111.025) (width 0.2) (layer "F.Cu") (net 12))
 (segment (start 108.855252 110.699748) (end 108.83 110.725) (width 0.2) (layer "F.Cu") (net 12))
 (segment (start 110.17112 110.699748) (end 108.855252 110.699748) (width 0.2) (layer "F.Cu") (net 12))
 (segment (start 110.17112 111.199874) (end 109.645126 111.199874) (width 0.2) (layer "F.Cu") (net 13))
 (segment (start 109.645126 111.199874) (end 108.83 112.015) (width 0.2) (layer "F.Cu") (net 13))
 (segment (start 108.83 112.015) (end 108.83 112.02) (width 0.2) (layer "F.Cu") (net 13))
 (segment (start 111.216447 112.477493) (end 111.216447 111.745075) (width 0.2) (layer "F.Cu") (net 7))
 (segment (start 111.169613 112.524327) (end 111.216447 112.477493) (width 0.2) (layer "F.Cu") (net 7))
 (via (at 111.169613 112.524327) (size 0.6) (drill 0.2) (layers "F.Cu" "B.Cu") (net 7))
 (segment (start 117.071 112.1161) (end 118.0161 111.171) (width 0.2) (layer "B.Cu") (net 7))
 (segment (start 113.1661 112.351) (end 116.5039 112.351) (width 0.2) (layer "B.Cu") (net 7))
 (segment (start 112.52 112.095) (end 112.775 112.35) (width 0.2) (layer "B.Cu") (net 7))
 (segment (start 118.251 110.6039) (end 118.251 110.494) (width 0.2) (layer "B.Cu") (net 7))
 (segment (start 112.775 112.35) (end 112.8329 112.35) (width 0.2) (layer "B.Cu") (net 7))
 (segment (start 111.169613 112.524327) (end 111.169613 112.400387) (width 0.2) (layer "B.Cu") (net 7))
 (segment (start 118.251 110.9361) (end 118.251 110.6039) (width 0.2) (layer "B.Cu") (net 7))
 (segment (start 118.251 110.494) (end 119.825 108.92) (width 0.2) (layer "B.Cu") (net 7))
 (segment (start 116.8361 112.351) (end 117.071 112.1161) (width 0.2) (layer "B.Cu") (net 7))
 (segment (start 118.0161 111.171) (end 118.251 110.9361) (width 0.2) (layer "B.Cu") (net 7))
 (segment (start 116.5039 112.351) (end 116.8361 112.351) (width 0.2) (layer "B.Cu") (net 7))
 (segment (start 111.169613 112.400387) (end 111.475 112.095) (width 0.2) (layer "B.Cu") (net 7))
 (segment (start 112.8329 112.35) (end 112.8339 112.351) (width 0.2) (layer "B.Cu") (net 7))
 (segment (start 111.475 112.095) (end 112.52 112.095) (width 0.2) (layer "B.Cu") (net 7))
 (segment (start 112.8339 112.351) (end 113.1661 112.351) (width 0.2) (layer "B.Cu") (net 7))
 (segment (start 111.95 112.7) (end 111.925 112.675) (width 0.2) (layer "F.Cu") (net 8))
 (segment (start 111.925 112.675) (end 111.925 112.37) (width 0.2) (layer "F.Cu") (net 8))
 (segment (start 111.675 111.745) (end 111.670453 111.740453) (width 0.2) (layer "F.Cu") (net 8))
 (segment (start 111.675 112.12) (end 111.675 111.745) (width 0.2) (layer "F.Cu") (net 8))
 (segment (start 111.925 112.37) (end 111.675 112.12) (width 0.2) (layer "F.Cu") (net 8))
 (via (at 111.95 112.7) (size 0.6) (drill 0.2) (layers "F.Cu" "B.Cu") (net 8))
 (segment (start 112 112.75) (end 112.6079 112.75) (width 0.2) (layer "B.Cu") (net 8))
 (segment (start 112.6079 112.75) (end 112.6089 112.751) (width 0.2) (layer "B.Cu") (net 8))
 (segment (start 111.95 112.7) (end 112 112.75) (width 0.2) (layer "B.Cu") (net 8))
 (segment (start 118.444 112.751) (end 119.735 111.46) (width 0.2) (layer "B.Cu") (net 8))
 (segment (start 112.6089 112.751) (end 118.444 112.751) (width 0.2) (layer "B.Cu") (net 8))
 (segment (start 119.735 111.46) (end 119.825 111.46) (width 0.2) (layer "B.Cu") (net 8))
 (segment (start 110.186831 112.637958) (end 110.196926 112.637958) (width 0.2) (layer "F.Cu") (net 6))
 (segment (start 110.425 112.347256) (end 110.716321 112.055935) (width 0.2) (layer "F.Cu") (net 6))
 (segment (start 110.716321 112.055935) (end 110.716321 111.745075) (width 0.2) (layer "F.Cu") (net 6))
 (segment (start 110.425 112.409884) (end 110.425 112.347256) (width 0.2) (layer "F.Cu") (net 6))
 (segment (start 110.196926 112.637958) (end 110.425 112.409884) (width 0.2) (layer "F.Cu") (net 6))
 (via (at 110.186831 112.637958) (size 0.6) (drill 0.2) (layers "F.Cu" "B.Cu") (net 6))
 (segment (start 110.196926 112.637958) (end 110.225 112.609884) (width 0.2) (layer "B.Cu") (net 6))
 (segment (start 117.85 108.355) (end 119.825 106.38) (width 0.2) (layer "B.Cu") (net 6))
 (segment (start 110.9 111.47) (end 112.52 111.47) (width 0.2) (layer "B.Cu") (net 6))
 (segment (start 117.85 110.77) (end 117.85 108.355) (width 0.2) (layer "B.Cu") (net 6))
 (segment (start 113 111.95) (end 116.67 111.95) (width 0.2) (layer "B.Cu") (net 6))
 (segment (start 116.67 111.95) (end 117.85 110.77) (width 0.2) (layer "B.Cu") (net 6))
 (segment (start 110.225 112.609884) (end 110.225 112.145) (width 0.2) (layer "B.Cu") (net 6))
 (segment (start 110.225 112.145) (end 110.9 111.47) (width 0.2) (layer "B.Cu") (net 6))
 (segment (start 112.52 111.47) (end 113 111.95) (width 0.2) (layer "B.Cu") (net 6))
 (segment (start 110.186831 112.637958) (end 110.196926 112.637958) (width 0.2) (layer "B.Cu") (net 6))
 (segment (start 112.39 113.465) (end 112.35 113.465) (width 0.2) (layer "F.Cu") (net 9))
 (segment (start 111.185 113.885) (end 111.93 113.885) (width 0.2) (layer "F.Cu") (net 9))
 (segment (start 112.445 113.52) (end 112.39 113.465) (width 0.2) (layer "F.Cu") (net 9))
 (segment (start 113.875 113.725) (end 113.67 113.52) (width 0.2) (layer "F.Cu") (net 9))
 (segment (start 114.05 113.495) (end 114.05 113.995) (width 0.2) (layer "F.Cu") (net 9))
 (segment (start 113.67 113.52) (end 112.445 113.52) (width 0.2) (layer "F.Cu") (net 9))
 (segment (start 112.345393 112.24545) (end 112.80045 112.24545) (width 0.2) (layer "F.Cu") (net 9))
 (segment (start 112.170579 111.740453) (end 112.286975 111.740453) (width 0.2) (layer "F.Cu") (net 9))
 (segment (start 112.286975 111.740453) (end 112.286975 112.187032) (width 0.2) (layer "F.Cu") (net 9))
 (segment (start 114.645 115.045) (end 113.875 114.275) (width 0.2) (layer "F.Cu") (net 9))
 (segment (start 111.05 114.02) (end 111.185 113.885) (width 0.2) (layer "F.Cu") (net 9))
 (segment (start 112.80045 112.24545) (end 114.05 113.495) (width 0.2) (layer "F.Cu") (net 9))
 (segment (start 113.875 114.275) (end 113.875 113.725) (width 0.2) (layer "F.Cu") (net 9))
 (segment (start 111.93 113.885) (end 112.35 113.465) (width 0.2) (layer "F.Cu") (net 9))
 (segment (start 119.825 114) (end 118.78 115.045) (width 0.2) (layer "F.Cu") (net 9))
 (segment (start 112.286975 112.187032) (end 112.345393 112.24545) (width 0.2) (layer "F.Cu") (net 9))
 (segment (start 118.78 115.045) (end 114.645 115.045) (width 0.2) (layer "F.Cu") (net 9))
 (segment (start 115.175 113.325) (end 115.175 113.725) (width 0.2) (layer "F.Cu") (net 14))
 (segment (start 114.1 112.095) (end 114.1 112.25) (width 0.2) (layer "F.Cu") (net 14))
 (segment (start 112.7619 110.699748) (end 112.816648 110.645) (width 0.2) (layer "F.Cu") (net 14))
 (segment (start 113.75 110.645) (end 114.1 110.995) (width 0.2) (layer "F.Cu") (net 14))
 (segment (start 114.1 112.229744) (end 114.1 112.095) (width 0.2) (layer "F.Cu") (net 14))
 (segment (start 115.35 113.479744) (end 114.1 112.229744) (width 0.2) (layer "F.Cu") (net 14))
 (segment (start 114.1 110.995) (end 114.1 112.095) (width 0.2) (layer "F.Cu") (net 14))
 (segment (start 115.35 113.995) (end 115.35 113.479744) (width 0.2) (layer "F.Cu") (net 14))
 (segment (start 112.816648 110.645) (end 113.75 110.645) (width 0.2) (layer "F.Cu") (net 14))
 (segment (start 105.55 108.885) (end 105.575 108.86) (width 0.2) (layer "F.Cu") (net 1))
 (segment (start 107.865 110.025) (end 106.465 110.025) (width 0.2) (layer "F.Cu") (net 1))
 (segment (start 107.87 110.02) (end 107.865 110.025) (width 0.2) (layer "F.Cu") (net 1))
 (segment (start 106.465 110.025) (end 105.55 109.11) (width 0.2) (layer "F.Cu") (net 1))
 (segment (start 105.55 109.11) (end 105.55 108.885) (width 0.2) (layer "F.Cu") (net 1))
 (segment (start 106.675 111.295) (end 105.68 111.295) (width 0.2) (layer "F.Cu") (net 17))
 (segment (start 107.87 111.025) (end 106.945 111.025) (width 0.2) (layer "F.Cu") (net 17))
 (segment (start 105.68 111.295) (end 105.575 111.4) (width 0.2) (layer "F.Cu") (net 17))
 (segment (start 106.945 111.025) (end 106.675 111.295) (width 0.2) (layer "F.Cu") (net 17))
 (segment (start 107.865 112.03) (end 105.955 113.94) (width 0.2) (layer "F.Cu") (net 18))
 (segment (start 105.955 113.94) (end 105.575 113.94) (width 0.2) (layer "F.Cu") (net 18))
 (segment (start 107.87 112.02) (end 107.865 112.025) (width 0.2) (layer "F.Cu") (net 18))
 (segment (start 107.865 112.025) (end 107.865 112.03) (width 0.2) (layer "F.Cu") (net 18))
 (segment (start 105.55 106.345) (end 105.575 106.32) (width 0.2) (layer "F.Cu") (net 16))
 (segment (start 106.8 107.595) (end 105.55 106.345) (width 0.2) (layer "F.Cu") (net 16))
 (segment (start 107.87 109.025) (end 106.8 107.955) (width 0.2) (layer "F.Cu") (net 16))
 (segment (start 106.8 107.955) (end 106.8 107.595) (width 0.2) (layer "F.Cu") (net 16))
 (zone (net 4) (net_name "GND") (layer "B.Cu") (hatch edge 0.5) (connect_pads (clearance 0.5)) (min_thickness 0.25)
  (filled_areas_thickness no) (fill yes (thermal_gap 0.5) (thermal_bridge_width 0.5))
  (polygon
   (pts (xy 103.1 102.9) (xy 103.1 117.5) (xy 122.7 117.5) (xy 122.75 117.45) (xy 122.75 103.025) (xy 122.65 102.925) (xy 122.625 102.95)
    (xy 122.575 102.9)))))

